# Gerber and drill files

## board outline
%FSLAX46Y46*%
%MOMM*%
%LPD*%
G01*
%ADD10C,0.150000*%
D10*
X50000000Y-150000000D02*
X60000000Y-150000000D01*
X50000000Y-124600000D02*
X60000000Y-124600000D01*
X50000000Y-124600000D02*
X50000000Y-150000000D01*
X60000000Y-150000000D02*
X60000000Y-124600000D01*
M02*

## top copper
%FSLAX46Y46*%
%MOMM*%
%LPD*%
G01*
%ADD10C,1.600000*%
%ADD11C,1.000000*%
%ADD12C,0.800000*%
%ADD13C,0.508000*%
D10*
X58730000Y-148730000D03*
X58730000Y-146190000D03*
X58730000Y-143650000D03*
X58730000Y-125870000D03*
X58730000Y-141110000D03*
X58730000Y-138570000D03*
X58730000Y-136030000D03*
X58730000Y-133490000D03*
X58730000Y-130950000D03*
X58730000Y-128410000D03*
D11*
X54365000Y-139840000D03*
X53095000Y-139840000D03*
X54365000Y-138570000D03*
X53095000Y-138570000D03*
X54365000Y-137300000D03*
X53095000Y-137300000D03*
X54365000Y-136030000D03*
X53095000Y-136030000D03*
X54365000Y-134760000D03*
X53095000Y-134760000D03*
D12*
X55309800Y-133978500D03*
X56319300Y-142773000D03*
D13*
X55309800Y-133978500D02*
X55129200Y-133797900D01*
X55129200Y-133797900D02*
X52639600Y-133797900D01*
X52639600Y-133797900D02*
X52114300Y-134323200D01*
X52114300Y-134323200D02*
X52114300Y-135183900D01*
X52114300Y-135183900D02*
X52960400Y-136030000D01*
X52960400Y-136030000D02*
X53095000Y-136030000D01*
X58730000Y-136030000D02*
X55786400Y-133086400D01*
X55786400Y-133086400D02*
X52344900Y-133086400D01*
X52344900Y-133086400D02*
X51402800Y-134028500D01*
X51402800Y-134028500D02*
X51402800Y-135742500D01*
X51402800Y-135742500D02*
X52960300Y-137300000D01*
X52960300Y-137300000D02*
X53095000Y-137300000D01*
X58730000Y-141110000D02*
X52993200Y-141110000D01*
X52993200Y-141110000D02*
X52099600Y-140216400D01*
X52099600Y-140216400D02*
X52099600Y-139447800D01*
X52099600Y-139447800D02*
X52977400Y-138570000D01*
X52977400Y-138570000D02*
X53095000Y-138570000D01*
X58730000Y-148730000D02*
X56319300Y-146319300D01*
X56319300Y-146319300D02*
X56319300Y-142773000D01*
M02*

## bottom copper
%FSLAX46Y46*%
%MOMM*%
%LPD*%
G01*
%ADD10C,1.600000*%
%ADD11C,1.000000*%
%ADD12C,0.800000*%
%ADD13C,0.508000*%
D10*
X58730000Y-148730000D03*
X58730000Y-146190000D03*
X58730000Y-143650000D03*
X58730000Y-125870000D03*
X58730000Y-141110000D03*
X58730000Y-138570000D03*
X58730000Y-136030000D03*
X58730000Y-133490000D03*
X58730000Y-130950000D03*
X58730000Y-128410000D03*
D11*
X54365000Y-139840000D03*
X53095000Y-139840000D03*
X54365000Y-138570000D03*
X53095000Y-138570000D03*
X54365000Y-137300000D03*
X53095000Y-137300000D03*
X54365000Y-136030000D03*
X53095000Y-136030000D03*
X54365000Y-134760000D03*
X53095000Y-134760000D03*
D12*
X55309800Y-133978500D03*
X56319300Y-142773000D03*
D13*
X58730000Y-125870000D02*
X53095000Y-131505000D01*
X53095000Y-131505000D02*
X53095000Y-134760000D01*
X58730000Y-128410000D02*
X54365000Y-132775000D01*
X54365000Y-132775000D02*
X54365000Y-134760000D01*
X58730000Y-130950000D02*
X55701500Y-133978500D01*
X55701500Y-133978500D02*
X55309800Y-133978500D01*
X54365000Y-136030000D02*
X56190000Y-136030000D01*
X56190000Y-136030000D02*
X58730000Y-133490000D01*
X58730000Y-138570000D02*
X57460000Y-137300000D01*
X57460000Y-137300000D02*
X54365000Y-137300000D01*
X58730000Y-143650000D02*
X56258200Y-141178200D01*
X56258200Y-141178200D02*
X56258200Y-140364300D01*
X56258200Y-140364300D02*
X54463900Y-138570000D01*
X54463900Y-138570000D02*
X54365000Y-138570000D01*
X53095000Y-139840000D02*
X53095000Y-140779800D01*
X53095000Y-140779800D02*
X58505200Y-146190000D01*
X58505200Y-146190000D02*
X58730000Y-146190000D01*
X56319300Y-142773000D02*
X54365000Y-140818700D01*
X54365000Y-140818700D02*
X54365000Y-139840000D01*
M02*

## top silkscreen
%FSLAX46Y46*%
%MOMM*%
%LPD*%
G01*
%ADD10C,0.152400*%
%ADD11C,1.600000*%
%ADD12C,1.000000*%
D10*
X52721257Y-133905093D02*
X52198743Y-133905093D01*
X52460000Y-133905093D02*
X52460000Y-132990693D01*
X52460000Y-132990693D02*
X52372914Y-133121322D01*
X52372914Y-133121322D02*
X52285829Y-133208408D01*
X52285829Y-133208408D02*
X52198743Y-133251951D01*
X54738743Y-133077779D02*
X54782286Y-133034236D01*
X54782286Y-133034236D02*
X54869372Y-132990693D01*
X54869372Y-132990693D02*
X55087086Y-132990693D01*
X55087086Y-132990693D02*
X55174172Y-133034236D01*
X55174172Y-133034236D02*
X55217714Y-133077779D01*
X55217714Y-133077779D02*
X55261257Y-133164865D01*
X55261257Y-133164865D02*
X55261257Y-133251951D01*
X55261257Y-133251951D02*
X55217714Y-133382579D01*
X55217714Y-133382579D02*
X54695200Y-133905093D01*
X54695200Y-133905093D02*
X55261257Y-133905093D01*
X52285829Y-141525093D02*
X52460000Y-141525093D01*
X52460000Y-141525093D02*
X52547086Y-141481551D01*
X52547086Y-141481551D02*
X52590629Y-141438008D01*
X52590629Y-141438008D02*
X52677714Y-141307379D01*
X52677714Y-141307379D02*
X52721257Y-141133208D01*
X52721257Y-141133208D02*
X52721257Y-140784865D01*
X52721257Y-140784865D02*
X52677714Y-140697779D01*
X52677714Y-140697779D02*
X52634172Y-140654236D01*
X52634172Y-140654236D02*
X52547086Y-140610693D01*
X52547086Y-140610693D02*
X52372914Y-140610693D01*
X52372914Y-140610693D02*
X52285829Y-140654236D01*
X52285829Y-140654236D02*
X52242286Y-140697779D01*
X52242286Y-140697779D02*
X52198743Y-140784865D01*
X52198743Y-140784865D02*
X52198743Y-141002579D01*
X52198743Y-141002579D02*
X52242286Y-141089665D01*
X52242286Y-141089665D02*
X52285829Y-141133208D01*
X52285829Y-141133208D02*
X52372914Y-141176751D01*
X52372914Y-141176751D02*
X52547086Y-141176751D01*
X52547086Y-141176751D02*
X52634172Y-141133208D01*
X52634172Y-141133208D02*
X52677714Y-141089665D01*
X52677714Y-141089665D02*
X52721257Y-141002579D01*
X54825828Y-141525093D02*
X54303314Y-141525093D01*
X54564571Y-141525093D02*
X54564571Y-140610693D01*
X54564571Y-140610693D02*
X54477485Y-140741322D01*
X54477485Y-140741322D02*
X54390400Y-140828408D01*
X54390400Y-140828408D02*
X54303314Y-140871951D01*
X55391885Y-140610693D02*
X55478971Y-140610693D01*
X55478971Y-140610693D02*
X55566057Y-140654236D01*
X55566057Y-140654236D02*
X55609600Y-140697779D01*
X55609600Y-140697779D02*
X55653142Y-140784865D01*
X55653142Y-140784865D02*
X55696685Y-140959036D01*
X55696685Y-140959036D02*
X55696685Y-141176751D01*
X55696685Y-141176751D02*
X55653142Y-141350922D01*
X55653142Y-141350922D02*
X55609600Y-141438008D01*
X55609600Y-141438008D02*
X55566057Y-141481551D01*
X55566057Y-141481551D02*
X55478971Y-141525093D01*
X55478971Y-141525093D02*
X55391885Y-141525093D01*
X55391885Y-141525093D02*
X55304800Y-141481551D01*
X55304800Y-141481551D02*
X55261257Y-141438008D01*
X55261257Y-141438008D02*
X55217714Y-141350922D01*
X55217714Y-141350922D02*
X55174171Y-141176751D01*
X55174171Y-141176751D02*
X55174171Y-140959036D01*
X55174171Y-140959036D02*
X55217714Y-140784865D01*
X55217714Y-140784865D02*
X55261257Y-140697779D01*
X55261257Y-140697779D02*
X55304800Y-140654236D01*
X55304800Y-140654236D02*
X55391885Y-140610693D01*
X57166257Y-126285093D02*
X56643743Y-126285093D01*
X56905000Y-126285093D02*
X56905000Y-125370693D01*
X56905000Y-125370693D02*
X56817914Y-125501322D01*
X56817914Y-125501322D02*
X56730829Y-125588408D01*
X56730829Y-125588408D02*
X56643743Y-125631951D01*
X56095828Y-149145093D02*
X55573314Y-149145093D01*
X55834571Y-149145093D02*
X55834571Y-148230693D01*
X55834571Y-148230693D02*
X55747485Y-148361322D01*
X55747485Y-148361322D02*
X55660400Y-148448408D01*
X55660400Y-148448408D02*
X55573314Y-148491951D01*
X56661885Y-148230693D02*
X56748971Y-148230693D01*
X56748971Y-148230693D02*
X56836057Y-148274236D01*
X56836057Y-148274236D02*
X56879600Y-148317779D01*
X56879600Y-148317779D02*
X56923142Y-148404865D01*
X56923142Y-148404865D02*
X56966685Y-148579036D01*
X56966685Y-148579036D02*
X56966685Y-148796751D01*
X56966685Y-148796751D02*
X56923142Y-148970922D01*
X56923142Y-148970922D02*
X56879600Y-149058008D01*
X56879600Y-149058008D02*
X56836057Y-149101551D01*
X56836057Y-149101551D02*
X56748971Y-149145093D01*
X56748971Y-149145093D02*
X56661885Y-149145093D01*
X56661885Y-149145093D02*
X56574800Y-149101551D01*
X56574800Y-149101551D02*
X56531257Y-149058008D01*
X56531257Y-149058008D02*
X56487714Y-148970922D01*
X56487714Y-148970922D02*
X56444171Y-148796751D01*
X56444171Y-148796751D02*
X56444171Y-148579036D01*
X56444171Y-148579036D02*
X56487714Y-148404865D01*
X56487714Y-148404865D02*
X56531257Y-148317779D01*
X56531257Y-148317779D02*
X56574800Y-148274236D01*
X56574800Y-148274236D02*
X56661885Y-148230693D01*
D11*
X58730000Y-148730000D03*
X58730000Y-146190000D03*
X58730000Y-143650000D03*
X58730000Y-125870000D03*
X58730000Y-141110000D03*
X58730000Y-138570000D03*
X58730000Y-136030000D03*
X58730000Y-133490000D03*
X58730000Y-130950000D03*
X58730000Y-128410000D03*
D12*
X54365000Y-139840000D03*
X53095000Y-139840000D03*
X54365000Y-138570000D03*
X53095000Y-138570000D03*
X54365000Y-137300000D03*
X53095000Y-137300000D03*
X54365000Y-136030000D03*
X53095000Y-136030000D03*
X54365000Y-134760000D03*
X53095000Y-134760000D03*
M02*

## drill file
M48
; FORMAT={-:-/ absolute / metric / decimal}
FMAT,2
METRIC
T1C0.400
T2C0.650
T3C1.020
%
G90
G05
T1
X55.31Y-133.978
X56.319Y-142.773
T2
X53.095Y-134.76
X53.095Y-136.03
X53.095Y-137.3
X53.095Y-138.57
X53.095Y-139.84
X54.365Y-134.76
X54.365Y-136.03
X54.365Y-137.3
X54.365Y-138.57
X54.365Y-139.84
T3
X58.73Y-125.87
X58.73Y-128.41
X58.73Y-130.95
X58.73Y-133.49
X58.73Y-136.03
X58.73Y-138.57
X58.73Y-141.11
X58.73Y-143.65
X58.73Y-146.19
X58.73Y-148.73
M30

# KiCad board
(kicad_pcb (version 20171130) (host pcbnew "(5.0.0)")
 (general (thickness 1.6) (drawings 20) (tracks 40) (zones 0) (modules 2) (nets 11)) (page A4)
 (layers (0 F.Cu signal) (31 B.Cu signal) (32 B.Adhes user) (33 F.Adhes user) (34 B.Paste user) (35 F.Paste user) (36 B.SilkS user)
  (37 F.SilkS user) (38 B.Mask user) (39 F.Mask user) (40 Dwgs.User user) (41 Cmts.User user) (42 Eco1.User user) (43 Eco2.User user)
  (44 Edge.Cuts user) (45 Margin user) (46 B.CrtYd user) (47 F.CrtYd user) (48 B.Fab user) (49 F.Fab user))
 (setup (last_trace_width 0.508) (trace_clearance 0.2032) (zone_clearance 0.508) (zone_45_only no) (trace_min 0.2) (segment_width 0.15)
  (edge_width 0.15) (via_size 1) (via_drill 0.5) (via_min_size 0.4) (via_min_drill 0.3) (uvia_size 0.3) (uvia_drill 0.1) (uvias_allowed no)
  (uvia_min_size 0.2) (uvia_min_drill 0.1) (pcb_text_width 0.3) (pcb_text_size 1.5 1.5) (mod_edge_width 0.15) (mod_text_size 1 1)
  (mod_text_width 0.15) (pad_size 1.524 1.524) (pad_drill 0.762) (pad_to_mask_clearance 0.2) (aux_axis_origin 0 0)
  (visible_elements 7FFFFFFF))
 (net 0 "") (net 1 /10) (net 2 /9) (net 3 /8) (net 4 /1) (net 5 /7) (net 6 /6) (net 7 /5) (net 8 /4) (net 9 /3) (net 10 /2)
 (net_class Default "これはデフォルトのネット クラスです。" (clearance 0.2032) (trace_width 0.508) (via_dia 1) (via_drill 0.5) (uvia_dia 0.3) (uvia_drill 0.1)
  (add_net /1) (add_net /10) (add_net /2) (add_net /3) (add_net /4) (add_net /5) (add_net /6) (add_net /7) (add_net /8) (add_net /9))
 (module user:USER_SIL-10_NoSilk (layer F.Cu) (at 58.73 137.3 270)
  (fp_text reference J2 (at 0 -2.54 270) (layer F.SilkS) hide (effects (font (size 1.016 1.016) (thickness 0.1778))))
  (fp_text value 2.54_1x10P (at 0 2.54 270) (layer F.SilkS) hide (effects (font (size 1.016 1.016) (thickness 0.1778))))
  (pad 10 thru_hole circle (at 11.43 0 270) (size 1.6 1.6) (drill 1.02) (layers *.Cu *.Mask F.SilkS) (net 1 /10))
  (pad 9 thru_hole circle (at 8.89 0 270) (size 1.6 1.6) (drill 1.02) (layers *.Cu *.Mask F.SilkS) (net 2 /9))
  (pad 8 thru_hole circle (at 6.35 0 270) (size 1.6 1.6) (drill 1.02) (layers *.Cu *.Mask F.SilkS) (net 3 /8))
  (pad 1 thru_hole circle (at -11.43 0 270) (size 1.6 1.6) (drill 1.02) (layers *.Cu *.Mask F.SilkS) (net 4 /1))
  (pad 7 thru_hole circle (at 3.81 0 270) (size 1.6 1.6) (drill 1.02) (layers *.Cu *.Mask F.SilkS) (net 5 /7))
  (pad 6 thru_hole circle (at 1.27 0 270) (size 1.6 1.6) (drill 1.02) (layers *.Cu *.Mask F.SilkS) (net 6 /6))
  (pad 5 thru_hole circle (at -1.27 0 270) (size 1.6 1.6) (drill 1.02) (layers *.Cu *.Mask F.SilkS) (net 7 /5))
  (pad 4 thru_hole circle (at -3.81 0 270) (size 1.6 1.6) (drill 1.02) (layers *.Cu *.Mask F.SilkS) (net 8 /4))
  (pad 3 thru_hole circle (at -6.35 0 270) (size 1.6 1.6) (drill 1.02) (layers *.Cu *.Mask F.SilkS) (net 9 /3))
  (pad 2 thru_hole circle (at -8.89 0 270) (size 1.6 1.6) (drill 1.02) (layers *.Cu *.Mask F.SilkS) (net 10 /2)))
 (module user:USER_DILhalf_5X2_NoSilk (layer F.Cu) (at 53.73 137.3)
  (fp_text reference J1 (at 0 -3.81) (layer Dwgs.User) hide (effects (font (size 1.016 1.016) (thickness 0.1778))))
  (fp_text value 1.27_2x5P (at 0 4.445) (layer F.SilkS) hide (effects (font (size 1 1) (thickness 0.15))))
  (pad 10 thru_hole circle (at 0.635 2.54) (size 1 1) (drill 0.65) (layers *.Cu *.Mask F.SilkS) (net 1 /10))
  (pad 9 thru_hole circle (at -0.635 2.54) (size 1 1) (drill 0.65) (layers *.Cu *.Mask F.SilkS) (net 2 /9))
  (pad 8 thru_hole circle (at 0.635 1.27) (size 1 1) (drill 0.65) (layers *.Cu *.Mask F.SilkS) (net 3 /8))
  (pad 7 thru_hole circle (at -0.635 1.27) (size 1 1) (drill 0.65) (layers *.Cu *.Mask F.SilkS) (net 5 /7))
  (pad 6 thru_hole circle (at 0.635 0) (size 1 1) (drill 0.65) (layers *.Cu *.Mask F.SilkS) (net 6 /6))
  (pad 5 thru_hole circle (at -0.635 0) (size 1 1) (drill 0.65) (layers *.Cu *.Mask F.SilkS) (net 7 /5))
  (pad 4 thru_hole circle (at 0.635 -1.27) (size 1 1) (drill 0.65) (layers *.Cu *.Mask F.SilkS) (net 8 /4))
  (pad 3 thru_hole circle (at -0.635 -1.27) (size 1 1) (drill 0.65) (layers *.Cu *.Mask F.SilkS) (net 9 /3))
  (pad 2 thru_hole circle (at 0.635 -2.54) (size 1 1) (drill 0.65) (layers *.Cu *.Mask F.SilkS) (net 10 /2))
  (pad 1 thru_hole circle (at -0.635 -2.54) (size 1 1) (drill 0.65) (layers *.Cu *.Mask F.SilkS) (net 4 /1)))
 (gr_line (start 50 150) (end 60 150) (angle 90) (layer Edge.Cuts) (width 0.15))
 (gr_line (start 50 124.6) (end 60 124.6) (angle 90) (layer Edge.Cuts) (width 0.15))
 (gr_line (start 50 124.6) (end 50 150) (angle 90) (layer Edge.Cuts) (width 0.15))
 (gr_line (start 60 150) (end 60 124.6) (angle 90) (layer Edge.Cuts) (width 0.15))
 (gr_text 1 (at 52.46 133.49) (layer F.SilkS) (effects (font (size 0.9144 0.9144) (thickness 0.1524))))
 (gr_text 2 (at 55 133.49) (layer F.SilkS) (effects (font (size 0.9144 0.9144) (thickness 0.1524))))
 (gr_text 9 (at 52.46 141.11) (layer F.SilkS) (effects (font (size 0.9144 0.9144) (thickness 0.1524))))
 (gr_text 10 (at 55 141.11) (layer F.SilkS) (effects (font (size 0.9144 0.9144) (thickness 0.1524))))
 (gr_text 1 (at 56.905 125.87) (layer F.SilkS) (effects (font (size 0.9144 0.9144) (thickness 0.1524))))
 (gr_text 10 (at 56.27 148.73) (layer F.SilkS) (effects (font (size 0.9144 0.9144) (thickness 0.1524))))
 (segment (start 58.73 125.87) (end 53.095 131.505) (width 0.508) (layer B.Cu) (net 4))
 (segment (start 53.095 131.505) (end 53.095 134.76) (width 0.508) (layer B.Cu) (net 4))
 (segment (start 58.73 128.41) (end 54.365 132.775) (width 0.508) (layer B.Cu) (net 10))
 (segment (start 54.365 132.775) (end 54.365 134.76) (width 0.508) (layer B.Cu) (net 10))
 (segment (start 55.3098 133.9785) (end 55.1292 133.7979) (width 0.508) (layer F.Cu) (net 9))
 (segment (start 55.1292 133.7979) (end 52.6396 133.7979) (width 0.508) (layer F.Cu) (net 9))
 (segment (start 52.6396 133.7979) (end 52.1143 134.3232) (width 0.508) (layer F.Cu) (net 9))
 (segment (start 52.1143 134.3232) (end 52.1143 135.1839) (width 0.508) (layer F.Cu) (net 9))
 (segment (start 52.1143 135.1839) (end 52.9604 136.03) (width 0.508) (layer F.Cu) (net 9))
 (segment (start 52.9604 136.03) (end 53.095 136.03) (width 0.508) (layer F.Cu) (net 9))
 (segment (start 58.73 130.95) (end 55.7015 133.9785) (width 0.508) (layer B.Cu) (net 9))
 (segment (start 55.7015 133.9785) (end 55.3098 133.9785) (width 0.508) (layer B.Cu) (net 9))
 (via (at 55.3098 133.9785) (size 0.8) (drill 0.4) (layers F.Cu B.Cu) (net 9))
 (segment (start 54.365 136.03) (end 56.19 136.03) (width 0.508) (layer B.Cu) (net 8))
 (segment (start 56.19 136.03) (end 58.73 133.49) (width 0.508) (layer B.Cu) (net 8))
 (segment (start 58.73 136.03) (end 55.7864 133.0864) (width 0.508) (layer F.Cu) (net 7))
 (segment (start 55.7864 133.0864) (end 52.3449 133.0864) (width 0.508) (layer F.Cu) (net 7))
 (segment (start 52.3449 133.0864) (end 51.4028 134.0285) (width 0.508) (layer F.Cu) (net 7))
 (segment (start 51.4028 134.0285) (end 51.4028 135.7425) (width 0.508) (layer F.Cu) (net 7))
 (segment (start 51.4028 135.7425) (end 52.9603 137.3) (width 0.508) (layer F.Cu) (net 7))
 (segment (start 52.9603 137.3) (end 53.095 137.3) (width 0.508) (layer F.Cu) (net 7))
 (segment (start 58.73 138.57) (end 57.46 137.3) (width 0.508) (layer B.Cu) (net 6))
 (segment (start 57.46 137.3) (end 54.365 137.3) (width 0.508) (layer B.Cu) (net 6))
 (segment (start 58.73 141.11) (end 52.9932 141.11) (width 0.508) (layer F.Cu) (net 5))
 (segment (start 52.9932 141.11) (end 52.0996 140.2164) (width 0.508) (layer F.Cu) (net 5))
 (segment (start 52.0996 140.2164) (end 52.0996 139.4478) (width 0.508) (layer F.Cu) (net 5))
 (segment (start 52.0996 139.4478) (end 52.9774 138.57) (width 0.508) (layer F.Cu) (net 5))
 (segment (start 52.9774 138.57) (end 53.095 138.57) (width 0.508) (layer F.Cu) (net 5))
 (segment (start 58.73 143.65) (end 56.2582 141.1782) (width 0.508) (layer B.Cu) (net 3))
 (segment (start 56.2582 141.1782) (end 56.2582 140.3643) (width 0.508) (layer B.Cu) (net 3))
 (segment (start 56.2582 140.3643) (end 54.4639 138.57) (width 0.508) (layer B.Cu) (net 3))
 (segment (start 54.4639 138.57) (end 54.365 138.57) (width 0.508) (layer B.Cu) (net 3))
 (segment (start 53.095 139.84) (end 53.095 140.7798) (width 0.508) (layer B.Cu) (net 2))
 (segment (start 53.095 140.7798) (end 58.5052 146.19) (width 0.508) (layer B.Cu) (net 2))
 (segment (start 58.5052 146.19) (end 58.73 146.19) (width 0.508) (layer B.Cu) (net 2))
 (segment (start 58.73 148.73) (end 56.3193 146.3193) (width 0.508) (layer F.Cu) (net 1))
 (segment (start 56.3193 146.3193) (end 56.3193 142.773) (width 0.508) (layer F.Cu) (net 1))
 (segment (start 56.3193 142.773) (end 54.365 140.8187) (width 0.508) (layer B.Cu) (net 1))
 (segment (start 54.365 140.8187) (end 54.365 139.84) (width 0.508) (layer B.Cu) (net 1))
 (via (at 56.3193 142.773) (size 0.8) (drill 0.4) (layers F.Cu B.Cu) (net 1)))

